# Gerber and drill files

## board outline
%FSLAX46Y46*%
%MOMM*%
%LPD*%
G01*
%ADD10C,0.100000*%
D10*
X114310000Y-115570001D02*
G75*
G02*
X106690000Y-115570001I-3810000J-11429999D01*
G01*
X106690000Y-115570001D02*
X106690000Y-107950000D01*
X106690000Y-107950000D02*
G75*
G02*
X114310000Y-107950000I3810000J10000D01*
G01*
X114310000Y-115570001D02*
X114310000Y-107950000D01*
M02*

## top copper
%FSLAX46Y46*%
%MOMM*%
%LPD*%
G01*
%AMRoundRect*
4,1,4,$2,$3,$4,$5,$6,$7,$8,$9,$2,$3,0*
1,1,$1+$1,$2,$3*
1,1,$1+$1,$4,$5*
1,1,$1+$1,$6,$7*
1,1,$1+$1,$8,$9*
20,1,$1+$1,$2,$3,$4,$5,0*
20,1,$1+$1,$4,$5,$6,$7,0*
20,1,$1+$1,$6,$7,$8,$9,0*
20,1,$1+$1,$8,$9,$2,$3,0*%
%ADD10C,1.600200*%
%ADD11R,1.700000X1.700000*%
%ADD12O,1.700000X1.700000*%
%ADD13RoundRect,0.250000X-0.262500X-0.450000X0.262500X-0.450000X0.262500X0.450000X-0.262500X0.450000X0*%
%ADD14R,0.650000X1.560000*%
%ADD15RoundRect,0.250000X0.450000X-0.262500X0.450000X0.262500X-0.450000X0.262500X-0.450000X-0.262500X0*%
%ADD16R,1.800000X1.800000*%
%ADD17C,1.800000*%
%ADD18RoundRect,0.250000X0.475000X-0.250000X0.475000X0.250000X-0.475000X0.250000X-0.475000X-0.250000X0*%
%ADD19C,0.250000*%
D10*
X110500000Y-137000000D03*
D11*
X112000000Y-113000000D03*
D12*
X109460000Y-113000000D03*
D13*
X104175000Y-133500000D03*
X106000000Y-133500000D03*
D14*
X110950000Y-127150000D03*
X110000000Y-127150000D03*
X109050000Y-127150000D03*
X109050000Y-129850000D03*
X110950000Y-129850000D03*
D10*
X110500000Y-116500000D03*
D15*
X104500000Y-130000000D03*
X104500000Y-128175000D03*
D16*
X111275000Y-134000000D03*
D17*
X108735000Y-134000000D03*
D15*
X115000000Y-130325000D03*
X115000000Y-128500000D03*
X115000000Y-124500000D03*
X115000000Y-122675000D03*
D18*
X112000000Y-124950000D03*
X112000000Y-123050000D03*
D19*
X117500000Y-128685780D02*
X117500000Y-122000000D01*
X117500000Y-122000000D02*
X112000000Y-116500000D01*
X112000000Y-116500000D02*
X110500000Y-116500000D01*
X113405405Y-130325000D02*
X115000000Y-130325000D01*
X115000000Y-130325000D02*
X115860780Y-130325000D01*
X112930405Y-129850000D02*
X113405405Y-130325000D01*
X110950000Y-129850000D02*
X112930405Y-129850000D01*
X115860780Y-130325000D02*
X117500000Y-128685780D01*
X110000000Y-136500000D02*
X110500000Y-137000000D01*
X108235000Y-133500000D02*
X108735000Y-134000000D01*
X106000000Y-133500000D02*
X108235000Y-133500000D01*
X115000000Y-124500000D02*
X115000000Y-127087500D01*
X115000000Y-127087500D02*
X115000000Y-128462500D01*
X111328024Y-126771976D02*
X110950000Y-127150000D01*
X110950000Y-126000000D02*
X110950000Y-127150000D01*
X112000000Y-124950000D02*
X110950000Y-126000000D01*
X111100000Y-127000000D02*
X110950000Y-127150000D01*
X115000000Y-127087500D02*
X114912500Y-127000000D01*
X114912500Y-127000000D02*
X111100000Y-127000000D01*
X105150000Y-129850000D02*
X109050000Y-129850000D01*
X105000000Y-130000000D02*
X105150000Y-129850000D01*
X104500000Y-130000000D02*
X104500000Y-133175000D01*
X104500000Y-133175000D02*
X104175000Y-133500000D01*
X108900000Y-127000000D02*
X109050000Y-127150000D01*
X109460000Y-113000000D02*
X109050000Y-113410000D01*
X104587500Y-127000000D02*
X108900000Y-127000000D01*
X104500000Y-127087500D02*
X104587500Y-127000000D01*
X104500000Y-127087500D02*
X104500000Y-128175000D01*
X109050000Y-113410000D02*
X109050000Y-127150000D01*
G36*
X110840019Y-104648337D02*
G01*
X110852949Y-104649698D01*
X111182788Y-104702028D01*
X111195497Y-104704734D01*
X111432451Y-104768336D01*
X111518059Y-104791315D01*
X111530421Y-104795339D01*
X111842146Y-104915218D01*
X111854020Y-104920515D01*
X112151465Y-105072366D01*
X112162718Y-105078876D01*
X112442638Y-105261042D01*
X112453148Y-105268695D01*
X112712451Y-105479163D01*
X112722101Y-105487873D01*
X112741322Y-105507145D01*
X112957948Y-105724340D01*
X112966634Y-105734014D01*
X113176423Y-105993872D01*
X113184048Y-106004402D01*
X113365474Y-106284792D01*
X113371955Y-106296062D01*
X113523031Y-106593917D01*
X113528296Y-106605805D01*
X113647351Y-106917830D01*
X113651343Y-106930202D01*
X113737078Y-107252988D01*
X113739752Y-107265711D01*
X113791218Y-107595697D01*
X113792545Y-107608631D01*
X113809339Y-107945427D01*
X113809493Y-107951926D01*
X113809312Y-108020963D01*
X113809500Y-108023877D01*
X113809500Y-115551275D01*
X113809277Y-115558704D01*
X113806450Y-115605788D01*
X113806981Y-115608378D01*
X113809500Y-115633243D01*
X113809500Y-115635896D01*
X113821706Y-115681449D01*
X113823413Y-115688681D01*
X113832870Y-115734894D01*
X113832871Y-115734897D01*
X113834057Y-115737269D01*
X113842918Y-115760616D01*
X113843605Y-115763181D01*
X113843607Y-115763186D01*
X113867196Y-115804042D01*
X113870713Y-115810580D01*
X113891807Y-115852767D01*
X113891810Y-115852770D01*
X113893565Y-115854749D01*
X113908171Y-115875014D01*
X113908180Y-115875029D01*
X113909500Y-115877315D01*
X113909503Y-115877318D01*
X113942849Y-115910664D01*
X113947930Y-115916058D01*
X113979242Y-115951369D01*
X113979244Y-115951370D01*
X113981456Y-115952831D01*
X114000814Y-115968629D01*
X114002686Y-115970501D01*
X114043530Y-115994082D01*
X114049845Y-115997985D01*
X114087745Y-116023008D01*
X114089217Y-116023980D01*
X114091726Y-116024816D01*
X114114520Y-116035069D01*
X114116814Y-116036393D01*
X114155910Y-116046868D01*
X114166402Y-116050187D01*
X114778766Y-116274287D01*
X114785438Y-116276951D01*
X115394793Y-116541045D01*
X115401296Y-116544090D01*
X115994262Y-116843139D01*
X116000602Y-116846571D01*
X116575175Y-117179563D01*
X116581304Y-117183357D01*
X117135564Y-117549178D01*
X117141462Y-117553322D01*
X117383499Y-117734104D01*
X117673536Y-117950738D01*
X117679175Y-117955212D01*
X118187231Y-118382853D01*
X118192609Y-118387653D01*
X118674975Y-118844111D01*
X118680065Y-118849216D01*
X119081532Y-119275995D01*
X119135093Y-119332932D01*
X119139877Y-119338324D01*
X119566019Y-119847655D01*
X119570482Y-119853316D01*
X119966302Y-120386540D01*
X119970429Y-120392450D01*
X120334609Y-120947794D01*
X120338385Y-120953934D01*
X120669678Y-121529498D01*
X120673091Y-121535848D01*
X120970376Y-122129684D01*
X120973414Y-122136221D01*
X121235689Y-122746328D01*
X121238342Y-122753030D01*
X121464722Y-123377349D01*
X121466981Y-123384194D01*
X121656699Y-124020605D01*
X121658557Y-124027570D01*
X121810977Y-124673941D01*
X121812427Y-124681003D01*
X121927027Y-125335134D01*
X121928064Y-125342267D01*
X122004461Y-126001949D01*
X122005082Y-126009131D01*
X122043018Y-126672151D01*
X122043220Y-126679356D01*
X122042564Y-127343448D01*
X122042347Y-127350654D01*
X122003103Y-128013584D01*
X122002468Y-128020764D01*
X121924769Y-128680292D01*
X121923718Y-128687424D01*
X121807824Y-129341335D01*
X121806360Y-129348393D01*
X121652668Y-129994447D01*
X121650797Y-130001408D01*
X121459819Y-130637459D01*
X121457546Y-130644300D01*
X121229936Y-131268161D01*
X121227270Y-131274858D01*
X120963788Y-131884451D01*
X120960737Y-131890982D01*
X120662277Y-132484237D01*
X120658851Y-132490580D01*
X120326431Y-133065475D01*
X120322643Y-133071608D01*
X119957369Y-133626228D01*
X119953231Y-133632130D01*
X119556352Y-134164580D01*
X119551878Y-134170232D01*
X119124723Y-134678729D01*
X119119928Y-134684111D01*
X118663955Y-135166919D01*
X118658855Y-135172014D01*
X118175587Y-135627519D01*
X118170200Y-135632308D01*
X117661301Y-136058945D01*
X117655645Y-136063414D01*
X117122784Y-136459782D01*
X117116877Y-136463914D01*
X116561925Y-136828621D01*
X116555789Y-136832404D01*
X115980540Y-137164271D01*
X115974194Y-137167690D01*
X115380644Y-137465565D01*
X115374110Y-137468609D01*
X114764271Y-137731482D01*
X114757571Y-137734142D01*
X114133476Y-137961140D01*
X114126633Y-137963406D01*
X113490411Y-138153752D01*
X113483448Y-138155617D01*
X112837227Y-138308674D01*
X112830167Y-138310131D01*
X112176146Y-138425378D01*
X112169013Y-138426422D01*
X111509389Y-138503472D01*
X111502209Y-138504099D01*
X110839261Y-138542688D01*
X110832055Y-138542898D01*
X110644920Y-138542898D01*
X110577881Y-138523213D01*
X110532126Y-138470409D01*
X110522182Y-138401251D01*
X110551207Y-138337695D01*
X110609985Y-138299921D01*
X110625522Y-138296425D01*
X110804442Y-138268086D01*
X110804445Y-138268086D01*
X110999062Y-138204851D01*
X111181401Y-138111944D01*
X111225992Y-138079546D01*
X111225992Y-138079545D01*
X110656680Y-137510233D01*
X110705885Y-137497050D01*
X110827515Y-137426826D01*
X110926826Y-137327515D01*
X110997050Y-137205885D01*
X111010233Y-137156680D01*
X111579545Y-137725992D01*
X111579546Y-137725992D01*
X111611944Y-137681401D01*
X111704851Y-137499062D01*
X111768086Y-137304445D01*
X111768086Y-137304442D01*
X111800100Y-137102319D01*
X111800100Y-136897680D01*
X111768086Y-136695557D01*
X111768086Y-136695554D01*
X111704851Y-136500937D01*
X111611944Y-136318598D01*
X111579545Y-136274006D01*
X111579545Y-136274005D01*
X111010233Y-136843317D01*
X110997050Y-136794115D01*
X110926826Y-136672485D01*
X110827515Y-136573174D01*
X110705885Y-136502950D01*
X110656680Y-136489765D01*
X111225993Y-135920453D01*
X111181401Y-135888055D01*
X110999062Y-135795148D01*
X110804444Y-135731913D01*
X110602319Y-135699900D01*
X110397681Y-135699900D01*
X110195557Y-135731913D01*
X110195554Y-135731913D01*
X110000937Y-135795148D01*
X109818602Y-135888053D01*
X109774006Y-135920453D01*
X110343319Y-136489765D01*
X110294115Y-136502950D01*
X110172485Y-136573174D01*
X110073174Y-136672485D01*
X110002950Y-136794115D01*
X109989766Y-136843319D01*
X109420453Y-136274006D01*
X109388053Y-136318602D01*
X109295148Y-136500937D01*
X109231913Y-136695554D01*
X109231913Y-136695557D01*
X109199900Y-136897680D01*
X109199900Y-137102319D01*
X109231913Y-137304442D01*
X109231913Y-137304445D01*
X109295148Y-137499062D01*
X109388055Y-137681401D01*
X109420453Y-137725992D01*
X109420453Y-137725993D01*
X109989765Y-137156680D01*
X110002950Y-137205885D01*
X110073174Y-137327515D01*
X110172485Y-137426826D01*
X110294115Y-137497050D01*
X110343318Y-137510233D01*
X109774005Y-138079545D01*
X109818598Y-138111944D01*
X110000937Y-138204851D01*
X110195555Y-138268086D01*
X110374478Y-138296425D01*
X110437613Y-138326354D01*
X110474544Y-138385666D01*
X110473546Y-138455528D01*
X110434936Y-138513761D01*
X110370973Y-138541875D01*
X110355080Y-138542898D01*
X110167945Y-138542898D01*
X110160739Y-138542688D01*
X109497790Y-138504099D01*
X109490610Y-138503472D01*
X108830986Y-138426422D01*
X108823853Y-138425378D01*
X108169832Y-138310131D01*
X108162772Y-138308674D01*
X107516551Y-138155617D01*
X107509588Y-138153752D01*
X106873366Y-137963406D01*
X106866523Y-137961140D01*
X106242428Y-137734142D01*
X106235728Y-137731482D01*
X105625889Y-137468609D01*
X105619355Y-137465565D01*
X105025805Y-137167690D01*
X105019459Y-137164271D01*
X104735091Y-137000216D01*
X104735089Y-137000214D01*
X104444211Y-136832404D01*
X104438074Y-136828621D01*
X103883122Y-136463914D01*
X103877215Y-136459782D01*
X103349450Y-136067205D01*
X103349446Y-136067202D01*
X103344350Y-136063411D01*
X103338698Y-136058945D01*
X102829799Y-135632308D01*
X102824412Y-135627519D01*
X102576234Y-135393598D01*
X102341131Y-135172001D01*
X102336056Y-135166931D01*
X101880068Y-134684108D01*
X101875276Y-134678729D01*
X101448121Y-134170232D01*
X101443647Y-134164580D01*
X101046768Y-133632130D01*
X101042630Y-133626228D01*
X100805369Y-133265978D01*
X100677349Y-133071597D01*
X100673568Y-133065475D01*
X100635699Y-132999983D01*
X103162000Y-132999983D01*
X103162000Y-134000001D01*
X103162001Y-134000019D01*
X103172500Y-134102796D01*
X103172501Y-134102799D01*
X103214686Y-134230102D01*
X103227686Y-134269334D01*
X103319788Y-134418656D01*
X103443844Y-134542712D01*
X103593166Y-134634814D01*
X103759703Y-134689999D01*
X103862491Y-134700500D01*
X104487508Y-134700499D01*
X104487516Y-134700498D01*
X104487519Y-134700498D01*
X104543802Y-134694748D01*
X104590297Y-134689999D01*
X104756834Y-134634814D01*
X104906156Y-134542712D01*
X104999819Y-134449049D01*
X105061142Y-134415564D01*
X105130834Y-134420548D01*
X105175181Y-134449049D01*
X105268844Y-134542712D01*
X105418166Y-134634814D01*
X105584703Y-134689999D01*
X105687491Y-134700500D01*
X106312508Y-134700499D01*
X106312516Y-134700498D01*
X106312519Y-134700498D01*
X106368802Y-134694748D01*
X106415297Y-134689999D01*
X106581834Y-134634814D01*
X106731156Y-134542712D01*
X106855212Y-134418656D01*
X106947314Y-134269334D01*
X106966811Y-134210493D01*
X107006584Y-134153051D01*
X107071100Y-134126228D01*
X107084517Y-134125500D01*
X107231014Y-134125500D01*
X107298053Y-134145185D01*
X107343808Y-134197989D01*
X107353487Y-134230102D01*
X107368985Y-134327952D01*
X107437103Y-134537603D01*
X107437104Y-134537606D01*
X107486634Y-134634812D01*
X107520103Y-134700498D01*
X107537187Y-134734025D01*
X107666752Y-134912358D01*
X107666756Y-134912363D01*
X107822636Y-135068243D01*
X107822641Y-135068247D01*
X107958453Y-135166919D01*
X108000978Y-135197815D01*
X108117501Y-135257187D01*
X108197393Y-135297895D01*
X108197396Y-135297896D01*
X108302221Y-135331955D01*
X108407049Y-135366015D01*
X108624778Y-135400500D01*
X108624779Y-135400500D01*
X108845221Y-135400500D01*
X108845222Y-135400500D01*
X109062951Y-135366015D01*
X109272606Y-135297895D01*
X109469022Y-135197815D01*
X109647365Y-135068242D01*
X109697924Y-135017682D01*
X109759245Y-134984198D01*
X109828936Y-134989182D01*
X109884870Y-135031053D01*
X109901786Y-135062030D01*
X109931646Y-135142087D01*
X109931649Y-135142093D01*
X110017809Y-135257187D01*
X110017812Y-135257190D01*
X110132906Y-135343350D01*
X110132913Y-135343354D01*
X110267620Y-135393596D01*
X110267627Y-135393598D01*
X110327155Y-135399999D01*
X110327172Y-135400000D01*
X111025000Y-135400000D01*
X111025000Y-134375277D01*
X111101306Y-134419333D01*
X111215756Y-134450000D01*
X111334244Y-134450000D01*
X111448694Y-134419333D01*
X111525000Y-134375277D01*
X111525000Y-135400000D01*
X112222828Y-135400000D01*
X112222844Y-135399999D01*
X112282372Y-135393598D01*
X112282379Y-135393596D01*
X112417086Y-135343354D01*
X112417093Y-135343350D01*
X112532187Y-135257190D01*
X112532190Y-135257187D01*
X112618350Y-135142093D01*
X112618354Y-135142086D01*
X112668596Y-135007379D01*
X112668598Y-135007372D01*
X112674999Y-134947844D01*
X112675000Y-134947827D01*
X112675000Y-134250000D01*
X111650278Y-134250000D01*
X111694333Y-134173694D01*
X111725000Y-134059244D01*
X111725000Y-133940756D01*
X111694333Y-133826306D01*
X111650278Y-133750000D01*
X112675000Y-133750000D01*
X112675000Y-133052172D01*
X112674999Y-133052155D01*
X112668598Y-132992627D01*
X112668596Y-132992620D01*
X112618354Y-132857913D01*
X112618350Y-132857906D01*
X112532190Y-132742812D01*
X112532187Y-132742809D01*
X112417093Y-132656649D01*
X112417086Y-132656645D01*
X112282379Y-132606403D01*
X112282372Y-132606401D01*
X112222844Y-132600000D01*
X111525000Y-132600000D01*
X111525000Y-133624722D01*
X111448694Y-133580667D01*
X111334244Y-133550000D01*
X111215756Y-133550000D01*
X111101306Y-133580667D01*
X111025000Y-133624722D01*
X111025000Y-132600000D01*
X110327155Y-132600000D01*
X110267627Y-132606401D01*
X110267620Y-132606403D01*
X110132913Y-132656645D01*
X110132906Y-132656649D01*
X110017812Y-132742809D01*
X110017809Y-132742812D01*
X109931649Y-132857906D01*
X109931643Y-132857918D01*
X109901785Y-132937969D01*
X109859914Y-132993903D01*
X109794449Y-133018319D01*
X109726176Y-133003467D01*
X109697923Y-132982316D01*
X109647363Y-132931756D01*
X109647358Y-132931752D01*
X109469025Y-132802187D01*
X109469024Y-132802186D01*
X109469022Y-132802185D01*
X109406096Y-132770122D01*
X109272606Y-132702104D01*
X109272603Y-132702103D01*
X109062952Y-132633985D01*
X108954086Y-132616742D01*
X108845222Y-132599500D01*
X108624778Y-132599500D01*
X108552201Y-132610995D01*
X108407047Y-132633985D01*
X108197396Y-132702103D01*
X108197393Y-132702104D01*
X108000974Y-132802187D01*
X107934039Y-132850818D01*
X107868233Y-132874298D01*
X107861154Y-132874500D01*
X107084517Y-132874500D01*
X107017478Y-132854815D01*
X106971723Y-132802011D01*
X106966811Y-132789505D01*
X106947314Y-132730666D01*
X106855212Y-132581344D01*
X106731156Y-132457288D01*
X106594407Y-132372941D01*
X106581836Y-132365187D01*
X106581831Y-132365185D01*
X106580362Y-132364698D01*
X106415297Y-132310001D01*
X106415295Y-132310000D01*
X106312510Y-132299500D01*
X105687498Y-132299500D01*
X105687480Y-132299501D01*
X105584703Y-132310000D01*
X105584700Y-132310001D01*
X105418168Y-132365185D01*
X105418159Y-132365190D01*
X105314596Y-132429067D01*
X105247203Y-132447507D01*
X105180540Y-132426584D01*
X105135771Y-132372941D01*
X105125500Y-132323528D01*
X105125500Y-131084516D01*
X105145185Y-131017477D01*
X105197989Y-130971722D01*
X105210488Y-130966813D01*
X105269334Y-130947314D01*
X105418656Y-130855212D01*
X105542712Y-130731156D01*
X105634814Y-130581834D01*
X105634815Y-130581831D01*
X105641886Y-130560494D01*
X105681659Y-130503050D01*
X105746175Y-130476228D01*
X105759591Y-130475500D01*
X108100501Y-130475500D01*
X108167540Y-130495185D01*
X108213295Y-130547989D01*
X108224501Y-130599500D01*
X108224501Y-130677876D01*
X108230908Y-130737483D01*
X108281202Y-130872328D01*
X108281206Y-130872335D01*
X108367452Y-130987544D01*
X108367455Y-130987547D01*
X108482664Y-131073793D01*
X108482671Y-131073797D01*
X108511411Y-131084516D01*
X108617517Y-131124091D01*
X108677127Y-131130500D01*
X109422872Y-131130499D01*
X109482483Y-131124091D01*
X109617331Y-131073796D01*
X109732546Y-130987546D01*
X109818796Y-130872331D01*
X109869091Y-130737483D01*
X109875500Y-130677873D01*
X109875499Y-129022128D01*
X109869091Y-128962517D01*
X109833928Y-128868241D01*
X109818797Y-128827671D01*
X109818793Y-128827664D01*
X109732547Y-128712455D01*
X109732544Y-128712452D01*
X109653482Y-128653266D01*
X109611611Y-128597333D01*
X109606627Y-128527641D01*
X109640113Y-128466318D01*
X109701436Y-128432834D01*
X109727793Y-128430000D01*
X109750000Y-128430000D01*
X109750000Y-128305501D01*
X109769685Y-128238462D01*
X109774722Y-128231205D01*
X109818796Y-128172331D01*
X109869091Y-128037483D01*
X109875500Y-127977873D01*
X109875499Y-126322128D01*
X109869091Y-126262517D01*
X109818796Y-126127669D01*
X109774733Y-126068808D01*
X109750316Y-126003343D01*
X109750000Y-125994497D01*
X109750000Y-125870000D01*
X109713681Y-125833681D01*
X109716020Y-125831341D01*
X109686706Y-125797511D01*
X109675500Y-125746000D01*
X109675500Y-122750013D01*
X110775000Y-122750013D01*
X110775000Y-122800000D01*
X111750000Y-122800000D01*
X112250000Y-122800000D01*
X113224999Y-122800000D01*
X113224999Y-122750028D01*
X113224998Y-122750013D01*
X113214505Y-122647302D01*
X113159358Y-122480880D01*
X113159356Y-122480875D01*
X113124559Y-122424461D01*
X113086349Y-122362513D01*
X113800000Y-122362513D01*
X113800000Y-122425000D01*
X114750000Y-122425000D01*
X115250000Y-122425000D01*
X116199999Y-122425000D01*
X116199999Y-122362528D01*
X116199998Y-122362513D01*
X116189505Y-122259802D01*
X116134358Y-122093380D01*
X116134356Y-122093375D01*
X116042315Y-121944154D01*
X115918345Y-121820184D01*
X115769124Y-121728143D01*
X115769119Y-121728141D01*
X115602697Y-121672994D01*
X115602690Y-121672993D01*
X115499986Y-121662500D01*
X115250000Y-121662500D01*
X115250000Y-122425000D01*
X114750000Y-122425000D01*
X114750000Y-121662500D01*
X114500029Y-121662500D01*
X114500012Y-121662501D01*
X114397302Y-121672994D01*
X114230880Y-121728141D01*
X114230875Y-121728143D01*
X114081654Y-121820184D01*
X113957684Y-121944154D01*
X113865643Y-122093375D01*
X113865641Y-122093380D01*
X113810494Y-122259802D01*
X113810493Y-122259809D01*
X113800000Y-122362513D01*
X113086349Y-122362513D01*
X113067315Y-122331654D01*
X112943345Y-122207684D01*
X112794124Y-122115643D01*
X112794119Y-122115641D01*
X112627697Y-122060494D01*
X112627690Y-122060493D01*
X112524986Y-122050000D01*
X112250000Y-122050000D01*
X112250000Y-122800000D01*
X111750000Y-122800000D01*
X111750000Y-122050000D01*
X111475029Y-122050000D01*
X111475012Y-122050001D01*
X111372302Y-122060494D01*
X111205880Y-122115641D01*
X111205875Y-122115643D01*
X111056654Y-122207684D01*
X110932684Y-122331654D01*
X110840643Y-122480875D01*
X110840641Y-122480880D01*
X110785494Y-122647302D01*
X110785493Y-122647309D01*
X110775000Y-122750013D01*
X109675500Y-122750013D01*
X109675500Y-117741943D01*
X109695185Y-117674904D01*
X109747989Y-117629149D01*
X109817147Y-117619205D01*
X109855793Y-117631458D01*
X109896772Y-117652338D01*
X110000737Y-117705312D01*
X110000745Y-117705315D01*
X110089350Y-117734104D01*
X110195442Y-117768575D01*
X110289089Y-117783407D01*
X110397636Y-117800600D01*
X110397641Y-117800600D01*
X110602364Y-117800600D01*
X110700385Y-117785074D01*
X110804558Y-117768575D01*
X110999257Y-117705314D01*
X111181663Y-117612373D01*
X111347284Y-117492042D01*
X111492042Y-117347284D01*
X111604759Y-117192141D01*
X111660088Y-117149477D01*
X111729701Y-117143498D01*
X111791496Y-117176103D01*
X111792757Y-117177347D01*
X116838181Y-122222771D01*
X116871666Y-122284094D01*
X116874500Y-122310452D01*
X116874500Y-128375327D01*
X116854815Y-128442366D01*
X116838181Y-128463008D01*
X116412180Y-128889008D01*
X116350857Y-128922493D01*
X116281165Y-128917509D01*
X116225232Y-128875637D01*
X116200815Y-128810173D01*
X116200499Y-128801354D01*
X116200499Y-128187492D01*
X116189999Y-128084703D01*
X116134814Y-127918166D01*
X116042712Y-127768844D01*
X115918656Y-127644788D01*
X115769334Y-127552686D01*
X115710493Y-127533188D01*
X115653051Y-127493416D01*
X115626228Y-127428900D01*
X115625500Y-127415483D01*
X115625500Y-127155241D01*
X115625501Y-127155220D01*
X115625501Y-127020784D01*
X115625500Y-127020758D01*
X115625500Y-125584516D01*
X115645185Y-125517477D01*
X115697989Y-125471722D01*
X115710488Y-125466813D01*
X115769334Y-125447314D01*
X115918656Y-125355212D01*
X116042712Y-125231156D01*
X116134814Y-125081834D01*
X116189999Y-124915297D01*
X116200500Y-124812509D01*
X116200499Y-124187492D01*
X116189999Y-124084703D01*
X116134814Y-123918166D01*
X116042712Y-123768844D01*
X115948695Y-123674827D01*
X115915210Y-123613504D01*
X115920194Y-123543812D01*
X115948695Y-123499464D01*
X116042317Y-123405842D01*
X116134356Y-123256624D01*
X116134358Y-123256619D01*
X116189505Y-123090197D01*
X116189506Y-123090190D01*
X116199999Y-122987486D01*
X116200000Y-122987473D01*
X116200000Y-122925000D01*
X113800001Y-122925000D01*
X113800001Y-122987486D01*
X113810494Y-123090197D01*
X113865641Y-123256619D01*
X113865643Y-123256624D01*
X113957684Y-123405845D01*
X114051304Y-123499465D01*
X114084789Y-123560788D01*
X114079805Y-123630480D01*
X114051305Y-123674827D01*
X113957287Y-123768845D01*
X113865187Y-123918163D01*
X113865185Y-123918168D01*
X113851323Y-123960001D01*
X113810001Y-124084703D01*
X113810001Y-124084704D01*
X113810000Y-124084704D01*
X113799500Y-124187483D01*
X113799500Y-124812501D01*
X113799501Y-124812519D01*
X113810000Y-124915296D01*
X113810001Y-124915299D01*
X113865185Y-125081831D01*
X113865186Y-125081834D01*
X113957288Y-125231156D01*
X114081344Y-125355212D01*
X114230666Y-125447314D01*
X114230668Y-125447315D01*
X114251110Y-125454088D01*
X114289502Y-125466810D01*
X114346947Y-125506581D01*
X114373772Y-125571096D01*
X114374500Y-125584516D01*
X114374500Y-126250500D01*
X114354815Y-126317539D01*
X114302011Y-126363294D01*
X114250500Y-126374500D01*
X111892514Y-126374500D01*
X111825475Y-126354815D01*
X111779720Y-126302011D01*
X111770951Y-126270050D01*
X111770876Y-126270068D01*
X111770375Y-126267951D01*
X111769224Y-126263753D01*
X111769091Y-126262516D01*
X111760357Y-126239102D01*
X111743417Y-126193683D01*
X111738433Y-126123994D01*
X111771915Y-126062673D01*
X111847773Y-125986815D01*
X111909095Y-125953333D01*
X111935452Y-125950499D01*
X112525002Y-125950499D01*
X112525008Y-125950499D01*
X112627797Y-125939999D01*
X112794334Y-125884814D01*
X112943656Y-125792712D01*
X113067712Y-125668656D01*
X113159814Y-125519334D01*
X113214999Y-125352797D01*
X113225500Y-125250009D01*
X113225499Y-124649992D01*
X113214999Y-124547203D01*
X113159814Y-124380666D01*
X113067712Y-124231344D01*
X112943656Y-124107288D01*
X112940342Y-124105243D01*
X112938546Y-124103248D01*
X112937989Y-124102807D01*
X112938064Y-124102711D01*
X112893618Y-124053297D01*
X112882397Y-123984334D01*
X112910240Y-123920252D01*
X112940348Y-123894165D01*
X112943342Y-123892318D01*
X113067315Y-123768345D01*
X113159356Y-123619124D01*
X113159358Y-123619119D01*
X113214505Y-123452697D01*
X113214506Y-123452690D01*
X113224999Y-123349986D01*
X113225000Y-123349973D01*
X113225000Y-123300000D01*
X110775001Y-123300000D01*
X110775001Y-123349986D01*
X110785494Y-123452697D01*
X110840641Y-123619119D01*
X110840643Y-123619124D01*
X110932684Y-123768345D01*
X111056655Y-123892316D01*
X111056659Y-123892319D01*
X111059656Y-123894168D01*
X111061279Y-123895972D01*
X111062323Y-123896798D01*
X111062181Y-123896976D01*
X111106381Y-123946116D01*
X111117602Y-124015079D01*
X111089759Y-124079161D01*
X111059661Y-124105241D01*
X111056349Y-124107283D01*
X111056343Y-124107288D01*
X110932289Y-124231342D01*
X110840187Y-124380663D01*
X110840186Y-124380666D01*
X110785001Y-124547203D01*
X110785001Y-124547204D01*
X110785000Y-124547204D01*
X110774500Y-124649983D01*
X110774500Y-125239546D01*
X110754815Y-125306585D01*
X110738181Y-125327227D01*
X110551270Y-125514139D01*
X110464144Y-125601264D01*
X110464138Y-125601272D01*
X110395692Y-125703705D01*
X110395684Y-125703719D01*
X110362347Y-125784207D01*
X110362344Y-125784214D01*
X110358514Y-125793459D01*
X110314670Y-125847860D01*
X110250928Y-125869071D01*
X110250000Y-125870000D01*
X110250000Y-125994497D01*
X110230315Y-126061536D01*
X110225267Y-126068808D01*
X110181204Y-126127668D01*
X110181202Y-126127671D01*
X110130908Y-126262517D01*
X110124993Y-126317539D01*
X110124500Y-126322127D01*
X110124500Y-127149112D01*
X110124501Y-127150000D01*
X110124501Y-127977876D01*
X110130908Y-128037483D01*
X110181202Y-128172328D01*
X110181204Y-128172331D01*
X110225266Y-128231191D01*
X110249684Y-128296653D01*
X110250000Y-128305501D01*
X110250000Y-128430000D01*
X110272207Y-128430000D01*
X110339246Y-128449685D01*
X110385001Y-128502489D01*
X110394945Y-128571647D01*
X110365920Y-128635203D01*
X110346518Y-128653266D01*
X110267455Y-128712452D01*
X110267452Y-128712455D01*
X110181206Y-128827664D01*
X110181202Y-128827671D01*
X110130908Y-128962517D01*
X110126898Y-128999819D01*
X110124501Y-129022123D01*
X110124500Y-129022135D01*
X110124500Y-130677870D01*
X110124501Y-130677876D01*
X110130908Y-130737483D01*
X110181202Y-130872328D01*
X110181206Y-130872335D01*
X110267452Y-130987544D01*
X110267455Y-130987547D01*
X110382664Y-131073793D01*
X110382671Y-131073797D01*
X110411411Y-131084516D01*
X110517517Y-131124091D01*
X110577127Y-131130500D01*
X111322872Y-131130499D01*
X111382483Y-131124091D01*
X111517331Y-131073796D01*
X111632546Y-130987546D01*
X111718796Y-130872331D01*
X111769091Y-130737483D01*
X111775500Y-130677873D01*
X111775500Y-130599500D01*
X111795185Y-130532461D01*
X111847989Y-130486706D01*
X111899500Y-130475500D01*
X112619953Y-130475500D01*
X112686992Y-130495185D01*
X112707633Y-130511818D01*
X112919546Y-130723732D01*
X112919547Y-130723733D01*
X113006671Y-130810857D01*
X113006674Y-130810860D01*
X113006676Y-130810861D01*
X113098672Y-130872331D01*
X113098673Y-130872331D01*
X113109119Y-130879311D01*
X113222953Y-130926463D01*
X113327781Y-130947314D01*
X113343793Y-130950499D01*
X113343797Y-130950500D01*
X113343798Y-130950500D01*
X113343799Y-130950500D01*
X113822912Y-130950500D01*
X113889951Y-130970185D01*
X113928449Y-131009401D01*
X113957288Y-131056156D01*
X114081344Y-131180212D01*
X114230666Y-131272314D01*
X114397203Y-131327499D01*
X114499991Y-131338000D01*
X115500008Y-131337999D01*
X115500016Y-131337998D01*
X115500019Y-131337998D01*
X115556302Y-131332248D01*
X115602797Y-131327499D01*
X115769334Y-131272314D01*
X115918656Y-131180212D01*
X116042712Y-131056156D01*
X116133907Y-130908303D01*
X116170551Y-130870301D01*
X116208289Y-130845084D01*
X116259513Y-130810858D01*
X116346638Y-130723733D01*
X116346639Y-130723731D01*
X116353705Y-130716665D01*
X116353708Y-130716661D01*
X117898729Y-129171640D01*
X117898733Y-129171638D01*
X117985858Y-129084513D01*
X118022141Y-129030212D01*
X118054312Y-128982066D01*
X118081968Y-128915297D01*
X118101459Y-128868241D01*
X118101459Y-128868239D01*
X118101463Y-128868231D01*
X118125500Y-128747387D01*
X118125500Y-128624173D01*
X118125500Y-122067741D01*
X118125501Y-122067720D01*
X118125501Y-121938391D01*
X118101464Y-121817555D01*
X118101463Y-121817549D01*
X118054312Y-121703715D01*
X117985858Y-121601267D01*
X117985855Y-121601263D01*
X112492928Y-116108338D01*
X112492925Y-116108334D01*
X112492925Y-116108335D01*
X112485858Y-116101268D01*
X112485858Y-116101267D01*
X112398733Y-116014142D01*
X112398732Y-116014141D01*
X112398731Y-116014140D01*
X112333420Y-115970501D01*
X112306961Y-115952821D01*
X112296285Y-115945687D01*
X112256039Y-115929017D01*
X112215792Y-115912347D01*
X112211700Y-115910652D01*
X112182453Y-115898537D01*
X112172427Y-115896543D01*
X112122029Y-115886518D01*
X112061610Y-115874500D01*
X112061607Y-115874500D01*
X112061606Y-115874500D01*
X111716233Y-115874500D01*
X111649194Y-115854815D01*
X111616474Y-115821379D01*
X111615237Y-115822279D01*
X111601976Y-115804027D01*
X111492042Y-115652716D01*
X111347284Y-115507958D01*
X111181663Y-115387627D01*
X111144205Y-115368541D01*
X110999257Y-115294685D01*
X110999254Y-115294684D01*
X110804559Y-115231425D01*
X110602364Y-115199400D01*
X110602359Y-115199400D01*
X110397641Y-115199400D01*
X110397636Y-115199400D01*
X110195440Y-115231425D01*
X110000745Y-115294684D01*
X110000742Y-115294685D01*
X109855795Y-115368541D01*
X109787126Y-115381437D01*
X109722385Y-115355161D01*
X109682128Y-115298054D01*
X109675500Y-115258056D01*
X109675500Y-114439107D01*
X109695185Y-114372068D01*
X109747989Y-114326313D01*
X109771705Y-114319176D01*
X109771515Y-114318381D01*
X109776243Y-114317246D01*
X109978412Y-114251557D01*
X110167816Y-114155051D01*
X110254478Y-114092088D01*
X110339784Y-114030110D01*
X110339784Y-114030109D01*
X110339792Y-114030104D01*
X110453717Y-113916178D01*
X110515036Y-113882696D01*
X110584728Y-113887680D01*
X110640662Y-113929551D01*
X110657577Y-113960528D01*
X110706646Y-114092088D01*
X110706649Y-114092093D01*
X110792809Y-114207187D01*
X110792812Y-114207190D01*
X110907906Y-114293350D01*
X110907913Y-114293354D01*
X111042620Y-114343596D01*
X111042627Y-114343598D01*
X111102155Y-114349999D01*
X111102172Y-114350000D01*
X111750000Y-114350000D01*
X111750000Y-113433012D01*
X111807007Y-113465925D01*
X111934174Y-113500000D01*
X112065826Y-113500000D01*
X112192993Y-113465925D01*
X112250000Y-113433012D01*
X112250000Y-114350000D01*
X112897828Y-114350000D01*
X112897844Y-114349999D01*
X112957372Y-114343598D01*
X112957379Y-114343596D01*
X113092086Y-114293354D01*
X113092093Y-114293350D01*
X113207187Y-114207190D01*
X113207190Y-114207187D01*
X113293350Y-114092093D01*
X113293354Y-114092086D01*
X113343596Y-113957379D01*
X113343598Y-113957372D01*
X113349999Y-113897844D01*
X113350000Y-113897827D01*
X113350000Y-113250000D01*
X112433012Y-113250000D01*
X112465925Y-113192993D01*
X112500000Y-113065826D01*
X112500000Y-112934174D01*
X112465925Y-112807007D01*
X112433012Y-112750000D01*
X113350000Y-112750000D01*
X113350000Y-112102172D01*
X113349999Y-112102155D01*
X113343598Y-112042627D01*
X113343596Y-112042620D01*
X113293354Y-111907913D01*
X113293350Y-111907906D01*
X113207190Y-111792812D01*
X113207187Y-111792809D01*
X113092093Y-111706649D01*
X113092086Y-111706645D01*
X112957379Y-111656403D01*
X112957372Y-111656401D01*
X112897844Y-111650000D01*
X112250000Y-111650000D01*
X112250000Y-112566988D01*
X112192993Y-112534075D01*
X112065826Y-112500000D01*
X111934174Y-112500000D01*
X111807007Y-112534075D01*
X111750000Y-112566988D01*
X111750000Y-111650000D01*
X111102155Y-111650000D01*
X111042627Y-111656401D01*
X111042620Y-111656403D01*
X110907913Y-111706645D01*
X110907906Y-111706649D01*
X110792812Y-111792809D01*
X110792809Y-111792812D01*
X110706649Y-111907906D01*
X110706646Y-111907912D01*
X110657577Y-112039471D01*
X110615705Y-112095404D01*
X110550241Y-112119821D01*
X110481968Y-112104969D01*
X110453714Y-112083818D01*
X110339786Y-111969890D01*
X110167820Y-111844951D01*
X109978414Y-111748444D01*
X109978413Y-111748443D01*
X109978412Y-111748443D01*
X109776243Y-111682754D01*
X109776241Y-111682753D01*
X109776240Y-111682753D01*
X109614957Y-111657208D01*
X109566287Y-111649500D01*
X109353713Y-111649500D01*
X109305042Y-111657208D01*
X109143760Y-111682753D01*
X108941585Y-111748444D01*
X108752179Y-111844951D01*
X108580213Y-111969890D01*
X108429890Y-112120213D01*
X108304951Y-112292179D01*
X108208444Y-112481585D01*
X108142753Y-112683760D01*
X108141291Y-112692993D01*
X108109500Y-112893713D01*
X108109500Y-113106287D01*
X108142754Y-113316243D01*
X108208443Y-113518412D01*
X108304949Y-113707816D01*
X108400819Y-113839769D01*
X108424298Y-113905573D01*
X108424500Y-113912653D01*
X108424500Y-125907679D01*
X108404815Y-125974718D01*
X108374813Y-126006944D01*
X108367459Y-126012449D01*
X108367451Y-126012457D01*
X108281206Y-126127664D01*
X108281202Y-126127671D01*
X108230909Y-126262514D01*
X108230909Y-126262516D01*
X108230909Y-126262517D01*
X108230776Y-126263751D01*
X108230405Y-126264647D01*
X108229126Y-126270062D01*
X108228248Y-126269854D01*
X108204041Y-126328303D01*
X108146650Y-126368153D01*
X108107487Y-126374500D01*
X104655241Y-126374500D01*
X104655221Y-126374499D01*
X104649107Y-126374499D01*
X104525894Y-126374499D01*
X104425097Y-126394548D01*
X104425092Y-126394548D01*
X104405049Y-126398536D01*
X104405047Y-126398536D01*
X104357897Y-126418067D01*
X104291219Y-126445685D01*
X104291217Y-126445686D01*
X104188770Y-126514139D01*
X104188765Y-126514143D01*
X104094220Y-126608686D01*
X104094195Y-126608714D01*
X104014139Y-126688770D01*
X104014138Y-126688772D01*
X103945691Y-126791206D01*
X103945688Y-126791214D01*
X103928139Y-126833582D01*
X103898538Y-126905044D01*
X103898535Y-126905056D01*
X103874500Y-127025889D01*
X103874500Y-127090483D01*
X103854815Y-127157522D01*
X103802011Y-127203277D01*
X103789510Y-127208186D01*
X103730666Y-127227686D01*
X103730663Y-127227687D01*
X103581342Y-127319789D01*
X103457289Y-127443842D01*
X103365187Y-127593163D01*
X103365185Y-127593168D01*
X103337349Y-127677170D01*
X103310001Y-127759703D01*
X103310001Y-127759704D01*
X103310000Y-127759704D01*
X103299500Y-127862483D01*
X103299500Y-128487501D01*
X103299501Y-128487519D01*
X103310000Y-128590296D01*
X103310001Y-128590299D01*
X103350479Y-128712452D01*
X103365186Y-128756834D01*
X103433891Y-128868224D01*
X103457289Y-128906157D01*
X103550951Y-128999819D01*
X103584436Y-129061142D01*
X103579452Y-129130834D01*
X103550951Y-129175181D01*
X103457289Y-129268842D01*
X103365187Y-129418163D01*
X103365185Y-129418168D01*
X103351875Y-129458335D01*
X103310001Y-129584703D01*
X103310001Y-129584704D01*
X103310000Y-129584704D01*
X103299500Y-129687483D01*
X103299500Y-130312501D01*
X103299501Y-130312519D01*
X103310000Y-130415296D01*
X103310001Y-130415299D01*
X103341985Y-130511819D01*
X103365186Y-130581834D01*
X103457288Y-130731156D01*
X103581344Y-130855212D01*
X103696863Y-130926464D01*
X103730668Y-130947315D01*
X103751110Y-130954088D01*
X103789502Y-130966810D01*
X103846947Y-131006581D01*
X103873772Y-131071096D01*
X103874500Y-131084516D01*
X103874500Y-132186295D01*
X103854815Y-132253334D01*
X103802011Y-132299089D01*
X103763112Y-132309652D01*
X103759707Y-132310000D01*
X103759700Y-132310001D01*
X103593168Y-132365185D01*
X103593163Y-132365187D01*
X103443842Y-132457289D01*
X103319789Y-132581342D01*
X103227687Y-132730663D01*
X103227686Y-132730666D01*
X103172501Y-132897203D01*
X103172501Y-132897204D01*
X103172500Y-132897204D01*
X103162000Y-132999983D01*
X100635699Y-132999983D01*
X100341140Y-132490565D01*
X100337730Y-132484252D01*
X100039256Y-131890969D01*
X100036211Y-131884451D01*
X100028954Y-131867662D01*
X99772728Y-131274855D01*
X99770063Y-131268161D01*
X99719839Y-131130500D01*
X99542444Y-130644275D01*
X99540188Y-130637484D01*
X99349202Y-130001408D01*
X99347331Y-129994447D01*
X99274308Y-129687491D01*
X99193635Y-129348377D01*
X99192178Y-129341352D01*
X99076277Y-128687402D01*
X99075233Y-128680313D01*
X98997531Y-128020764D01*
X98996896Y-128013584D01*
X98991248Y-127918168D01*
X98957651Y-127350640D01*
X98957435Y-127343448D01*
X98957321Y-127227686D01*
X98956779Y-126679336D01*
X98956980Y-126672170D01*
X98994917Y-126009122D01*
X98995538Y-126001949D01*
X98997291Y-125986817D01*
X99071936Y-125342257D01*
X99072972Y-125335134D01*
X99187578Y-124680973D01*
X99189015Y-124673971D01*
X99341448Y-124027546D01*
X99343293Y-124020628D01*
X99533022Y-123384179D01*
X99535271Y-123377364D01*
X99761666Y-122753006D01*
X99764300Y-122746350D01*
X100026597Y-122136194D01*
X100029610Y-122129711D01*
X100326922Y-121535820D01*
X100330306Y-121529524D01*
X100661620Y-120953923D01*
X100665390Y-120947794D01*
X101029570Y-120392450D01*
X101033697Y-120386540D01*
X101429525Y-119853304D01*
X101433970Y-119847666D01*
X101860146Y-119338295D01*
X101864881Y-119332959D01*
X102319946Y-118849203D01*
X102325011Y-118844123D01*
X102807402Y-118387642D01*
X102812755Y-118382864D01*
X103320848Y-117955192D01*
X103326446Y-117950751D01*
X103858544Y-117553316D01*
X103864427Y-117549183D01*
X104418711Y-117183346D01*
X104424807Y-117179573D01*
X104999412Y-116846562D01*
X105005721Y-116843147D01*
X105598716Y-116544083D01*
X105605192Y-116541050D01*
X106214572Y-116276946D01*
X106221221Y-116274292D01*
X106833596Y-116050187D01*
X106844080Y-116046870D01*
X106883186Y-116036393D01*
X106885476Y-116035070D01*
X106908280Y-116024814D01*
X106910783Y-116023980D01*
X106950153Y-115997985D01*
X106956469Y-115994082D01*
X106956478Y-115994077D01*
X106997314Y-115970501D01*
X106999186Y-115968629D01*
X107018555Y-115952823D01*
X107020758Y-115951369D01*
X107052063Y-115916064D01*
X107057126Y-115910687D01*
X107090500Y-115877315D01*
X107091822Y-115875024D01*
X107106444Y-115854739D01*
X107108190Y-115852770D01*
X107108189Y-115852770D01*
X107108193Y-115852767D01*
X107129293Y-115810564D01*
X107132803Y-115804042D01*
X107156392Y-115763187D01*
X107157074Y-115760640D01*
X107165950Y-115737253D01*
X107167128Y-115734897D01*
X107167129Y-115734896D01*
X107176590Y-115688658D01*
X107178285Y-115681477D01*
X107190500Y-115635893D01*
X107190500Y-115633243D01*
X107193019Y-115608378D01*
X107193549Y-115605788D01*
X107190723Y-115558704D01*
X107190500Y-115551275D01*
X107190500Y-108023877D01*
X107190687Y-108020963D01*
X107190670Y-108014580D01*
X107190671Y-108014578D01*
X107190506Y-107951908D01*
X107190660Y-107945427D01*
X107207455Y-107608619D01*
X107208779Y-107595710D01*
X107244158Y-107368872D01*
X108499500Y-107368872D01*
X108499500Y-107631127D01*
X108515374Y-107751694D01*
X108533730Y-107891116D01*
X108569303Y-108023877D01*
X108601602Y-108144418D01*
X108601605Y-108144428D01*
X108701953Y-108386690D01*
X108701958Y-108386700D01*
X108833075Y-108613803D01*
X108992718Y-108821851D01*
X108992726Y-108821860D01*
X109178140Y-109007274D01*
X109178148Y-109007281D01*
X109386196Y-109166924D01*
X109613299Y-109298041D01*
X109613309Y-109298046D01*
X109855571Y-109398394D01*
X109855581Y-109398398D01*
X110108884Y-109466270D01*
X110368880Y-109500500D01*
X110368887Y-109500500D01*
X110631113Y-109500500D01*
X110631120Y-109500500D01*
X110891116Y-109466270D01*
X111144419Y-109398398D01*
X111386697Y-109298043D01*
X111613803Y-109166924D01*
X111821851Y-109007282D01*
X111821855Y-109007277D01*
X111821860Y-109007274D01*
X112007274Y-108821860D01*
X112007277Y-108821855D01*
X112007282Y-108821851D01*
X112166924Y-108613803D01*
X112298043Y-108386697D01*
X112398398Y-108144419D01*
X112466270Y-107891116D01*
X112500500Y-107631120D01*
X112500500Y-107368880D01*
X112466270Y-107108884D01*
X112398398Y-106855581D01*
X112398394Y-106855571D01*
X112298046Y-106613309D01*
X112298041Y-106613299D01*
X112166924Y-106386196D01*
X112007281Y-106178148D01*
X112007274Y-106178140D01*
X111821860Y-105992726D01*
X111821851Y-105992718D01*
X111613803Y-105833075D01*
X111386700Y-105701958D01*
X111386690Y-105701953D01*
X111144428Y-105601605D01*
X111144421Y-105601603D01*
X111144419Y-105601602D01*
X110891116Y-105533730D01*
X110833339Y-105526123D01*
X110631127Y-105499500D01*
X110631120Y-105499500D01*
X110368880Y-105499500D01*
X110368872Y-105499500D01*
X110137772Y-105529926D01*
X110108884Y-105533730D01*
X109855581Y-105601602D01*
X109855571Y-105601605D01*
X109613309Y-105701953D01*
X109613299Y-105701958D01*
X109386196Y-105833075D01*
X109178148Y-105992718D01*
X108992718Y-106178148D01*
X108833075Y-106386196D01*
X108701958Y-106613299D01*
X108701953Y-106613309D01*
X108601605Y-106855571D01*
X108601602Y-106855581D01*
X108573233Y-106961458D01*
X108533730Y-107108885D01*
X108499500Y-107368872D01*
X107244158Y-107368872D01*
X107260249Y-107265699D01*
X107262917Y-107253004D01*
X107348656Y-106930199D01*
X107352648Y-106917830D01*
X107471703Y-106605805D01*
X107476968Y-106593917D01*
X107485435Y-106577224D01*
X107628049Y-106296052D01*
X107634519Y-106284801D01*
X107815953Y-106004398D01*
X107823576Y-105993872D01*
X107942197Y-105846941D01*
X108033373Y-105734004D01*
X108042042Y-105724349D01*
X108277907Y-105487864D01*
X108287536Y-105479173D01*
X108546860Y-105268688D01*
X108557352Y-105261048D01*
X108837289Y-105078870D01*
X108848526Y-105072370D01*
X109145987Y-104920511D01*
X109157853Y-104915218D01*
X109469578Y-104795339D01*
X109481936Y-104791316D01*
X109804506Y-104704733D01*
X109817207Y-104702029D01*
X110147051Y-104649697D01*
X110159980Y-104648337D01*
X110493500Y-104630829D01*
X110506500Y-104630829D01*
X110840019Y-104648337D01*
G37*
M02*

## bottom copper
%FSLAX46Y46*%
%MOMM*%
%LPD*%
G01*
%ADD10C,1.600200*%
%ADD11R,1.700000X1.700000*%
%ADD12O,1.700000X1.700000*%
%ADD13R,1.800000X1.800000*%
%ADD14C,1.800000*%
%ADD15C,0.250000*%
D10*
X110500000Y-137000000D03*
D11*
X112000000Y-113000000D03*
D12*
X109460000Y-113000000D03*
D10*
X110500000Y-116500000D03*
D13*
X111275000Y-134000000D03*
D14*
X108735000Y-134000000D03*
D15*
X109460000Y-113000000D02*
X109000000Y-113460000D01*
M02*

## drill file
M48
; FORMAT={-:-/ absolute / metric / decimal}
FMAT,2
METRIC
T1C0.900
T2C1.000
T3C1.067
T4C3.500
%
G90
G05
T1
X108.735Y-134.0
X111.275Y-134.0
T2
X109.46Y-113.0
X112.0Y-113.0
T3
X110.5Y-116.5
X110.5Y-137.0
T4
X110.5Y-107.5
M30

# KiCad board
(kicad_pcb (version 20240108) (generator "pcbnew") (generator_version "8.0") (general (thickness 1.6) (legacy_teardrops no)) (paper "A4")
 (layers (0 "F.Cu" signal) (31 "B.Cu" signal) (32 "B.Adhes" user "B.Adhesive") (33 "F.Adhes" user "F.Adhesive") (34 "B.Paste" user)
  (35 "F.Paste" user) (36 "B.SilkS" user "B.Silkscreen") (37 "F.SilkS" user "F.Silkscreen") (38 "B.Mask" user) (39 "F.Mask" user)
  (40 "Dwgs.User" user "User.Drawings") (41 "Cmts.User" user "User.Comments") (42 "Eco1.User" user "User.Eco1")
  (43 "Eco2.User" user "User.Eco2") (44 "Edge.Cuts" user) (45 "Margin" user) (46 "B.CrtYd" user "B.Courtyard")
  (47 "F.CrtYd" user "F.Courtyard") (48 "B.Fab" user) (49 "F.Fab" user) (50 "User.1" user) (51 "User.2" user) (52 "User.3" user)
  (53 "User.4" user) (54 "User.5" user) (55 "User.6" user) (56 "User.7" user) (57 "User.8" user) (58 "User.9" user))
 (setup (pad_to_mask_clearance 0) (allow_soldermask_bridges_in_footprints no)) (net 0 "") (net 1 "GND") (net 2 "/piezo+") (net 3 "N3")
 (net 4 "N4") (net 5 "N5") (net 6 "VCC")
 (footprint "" (layer "F.Cu") (at 110.5 137)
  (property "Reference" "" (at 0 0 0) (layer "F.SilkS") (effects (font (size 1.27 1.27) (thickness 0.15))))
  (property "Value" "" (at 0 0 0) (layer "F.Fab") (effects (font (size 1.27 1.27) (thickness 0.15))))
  (pad "2" thru_hole circle (at 0 0) (size 1.6002 1.6002) (drill 1.0668) (layers "*.Cu" "*.Mask") (remove_unused_layers no) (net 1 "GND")
   (solder_mask_margin 0.102)))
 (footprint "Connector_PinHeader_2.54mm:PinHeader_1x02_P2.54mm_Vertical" (layer "F.Cu") (at 112 113 -90)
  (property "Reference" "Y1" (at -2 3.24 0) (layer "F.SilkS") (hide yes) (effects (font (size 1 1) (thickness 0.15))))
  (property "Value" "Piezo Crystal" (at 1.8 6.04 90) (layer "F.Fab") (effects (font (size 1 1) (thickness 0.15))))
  (pad "1" thru_hole rect (at 0 0 270) (size 1.7 1.7) (drill 1) (layers "*.Cu" "*.Mask") (remove_unused_layers no) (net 1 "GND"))
  (pad "2" thru_hole oval (at 0 2.54 270) (size 1.7 1.7) (drill 1) (layers "*.Cu" "*.Mask") (remove_unused_layers no) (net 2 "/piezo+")))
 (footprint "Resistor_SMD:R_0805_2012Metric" (layer "F.Cu") (at 105.0875 133.5)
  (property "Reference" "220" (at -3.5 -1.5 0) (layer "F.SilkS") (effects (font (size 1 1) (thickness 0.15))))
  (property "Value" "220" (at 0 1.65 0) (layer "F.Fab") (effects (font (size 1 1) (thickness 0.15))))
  (pad "1" smd roundrect (at -0.9125 0) (size 1.025 1.4) (layers "F.Cu" "F.Paste" "F.Mask") (roundrect_rratio 0.243902439) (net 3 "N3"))
  (pad "2" smd roundrect (at 0.9125 0) (size 1.025 1.4) (layers "F.Cu" "F.Paste" "F.Mask") (roundrect_rratio 0.243902439) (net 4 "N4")))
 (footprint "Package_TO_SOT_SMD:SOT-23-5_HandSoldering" (layer "F.Cu") (at 110 128.5 -90)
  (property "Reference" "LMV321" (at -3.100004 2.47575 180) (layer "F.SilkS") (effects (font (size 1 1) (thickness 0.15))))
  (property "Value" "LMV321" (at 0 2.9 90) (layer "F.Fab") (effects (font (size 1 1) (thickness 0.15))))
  (pad "1" smd rect (at -1.35 -0.95 270) (size 1.56 0.65) (layers "F.Cu" "F.Paste" "F.Mask") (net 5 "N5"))
  (pad "2" smd rect (at -1.35 0 270) (size 1.56 0.65) (layers "F.Cu" "F.Paste" "F.Mask") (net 1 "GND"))
  (pad "3" smd rect (at -1.35 0.95 270) (size 1.56 0.65) (layers "F.Cu" "F.Paste" "F.Mask") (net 2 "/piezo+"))
  (pad "4" smd rect (at 1.35 0.95 270) (size 1.56 0.65) (layers "F.Cu" "F.Paste" "F.Mask") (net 3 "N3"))
  (pad "5" smd rect (at 1.35 -0.95 270) (size 1.56 0.65) (layers "F.Cu" "F.Paste" "F.Mask") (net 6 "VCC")))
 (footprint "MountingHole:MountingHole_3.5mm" (layer "F.Cu") (at 110.5 107.5)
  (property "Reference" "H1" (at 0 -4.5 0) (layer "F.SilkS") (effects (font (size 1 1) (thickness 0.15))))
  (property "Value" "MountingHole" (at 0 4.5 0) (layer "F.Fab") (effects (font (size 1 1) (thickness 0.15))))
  (pad "" np_thru_hole circle (at 0 0) (size 3.5 3.5) (drill 3.5) (layers "*.Cu" "*.Mask")))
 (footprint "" (layer "F.Cu") (at 110.5 116.5)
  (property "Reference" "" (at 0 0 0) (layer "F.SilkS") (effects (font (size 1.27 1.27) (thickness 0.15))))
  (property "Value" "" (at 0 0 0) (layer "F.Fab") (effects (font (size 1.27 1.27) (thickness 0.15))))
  (pad "1" thru_hole circle (at 0 0) (size 1.6002 1.6002) (drill 1.0668) (layers "*.Cu" "*.Mask") (remove_unused_layers no) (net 6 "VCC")
   (solder_mask_margin 0.102)))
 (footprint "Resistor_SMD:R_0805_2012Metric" (layer "F.Cu") (at 104.5 129.0875 90)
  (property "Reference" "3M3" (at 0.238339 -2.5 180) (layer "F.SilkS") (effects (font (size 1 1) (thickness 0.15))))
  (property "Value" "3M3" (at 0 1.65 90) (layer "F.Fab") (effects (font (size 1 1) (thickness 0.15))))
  (pad "1" smd roundrect (at -0.9125 0 90) (size 1.025 1.4) (layers "F.Cu" "F.Paste" "F.Mask") (roundrect_rratio 0.243902439) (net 3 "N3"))
  (pad "2" smd roundrect (at 0.9125 0 90) (size 1.025 1.4) (layers "F.Cu" "F.Paste" "F.Mask") (roundrect_rratio 0.243902439)
   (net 2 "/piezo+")))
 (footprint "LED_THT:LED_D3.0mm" (layer "F.Cu") (at 111.275 134 180)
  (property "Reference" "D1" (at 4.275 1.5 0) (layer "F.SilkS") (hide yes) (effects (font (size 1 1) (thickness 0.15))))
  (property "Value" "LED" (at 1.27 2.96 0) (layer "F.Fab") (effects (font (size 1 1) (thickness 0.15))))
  (pad "1" thru_hole rect (at 0 0 180) (size 1.8 1.8) (drill 0.9) (layers "*.Cu" "*.Mask") (remove_unused_layers no) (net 1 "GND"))
  (pad "2" thru_hole circle (at 2.54 0 180) (size 1.8 1.8) (drill 0.9) (layers "*.Cu" "*.Mask") (remove_unused_layers no) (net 4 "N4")))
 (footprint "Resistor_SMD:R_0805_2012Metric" (layer "F.Cu") (at 115 129.4125 90)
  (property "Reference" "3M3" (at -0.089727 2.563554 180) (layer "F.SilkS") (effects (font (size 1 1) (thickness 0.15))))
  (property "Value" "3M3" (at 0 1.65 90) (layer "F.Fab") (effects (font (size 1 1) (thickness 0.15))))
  (pad "1" smd roundrect (at -0.9125 0 90) (size 1.025 1.4) (layers "F.Cu" "F.Paste" "F.Mask") (roundrect_rratio 0.243902439) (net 6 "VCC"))
  (pad "2" smd roundrect (at 0.9125 0 90) (size 1.025 1.4) (layers "F.Cu" "F.Paste" "F.Mask") (roundrect_rratio 0.243902439) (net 5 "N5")))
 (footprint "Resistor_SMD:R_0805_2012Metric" (layer "F.Cu") (at 115 123.5875 90)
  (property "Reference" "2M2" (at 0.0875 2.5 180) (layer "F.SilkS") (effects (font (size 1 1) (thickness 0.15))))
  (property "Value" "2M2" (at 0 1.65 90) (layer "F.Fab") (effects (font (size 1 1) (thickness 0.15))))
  (pad "1" smd roundrect (at -0.9125 0 90) (size 1.025 1.4) (layers "F.Cu" "F.Paste" "F.Mask") (roundrect_rratio 0.243902439) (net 5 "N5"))
  (pad "2" smd roundrect (at 0.9125 0 90) (size 1.025 1.4) (layers "F.Cu" "F.Paste" "F.Mask") (roundrect_rratio 0.243902439) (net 1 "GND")))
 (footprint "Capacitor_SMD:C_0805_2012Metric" (layer "F.Cu") (at 112 124 90)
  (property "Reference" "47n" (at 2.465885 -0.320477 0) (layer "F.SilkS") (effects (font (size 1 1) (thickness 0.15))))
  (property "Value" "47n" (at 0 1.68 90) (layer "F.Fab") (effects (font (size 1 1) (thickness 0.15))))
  (pad "1" smd roundrect (at -0.95 0 90) (size 1 1.45) (layers "F.Cu" "F.Paste" "F.Mask") (roundrect_rratio 0.25) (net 5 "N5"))
  (pad "2" smd roundrect (at 0.95 0 90) (size 1 1.45) (layers "F.Cu" "F.Paste" "F.Mask") (roundrect_rratio 0.25) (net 1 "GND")))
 (gr_arc (start 114.31 115.570001) (mid 110.5 139.048277) (end 106.69 115.570001) (stroke (width 0.1) (type default)) (layer "Edge.Cuts"))
 (gr_line (start 106.69 115.570001) (end 106.69 107.95) (stroke (width 0.1) (type default)) (layer "Edge.Cuts"))
 (gr_arc (start 106.69 107.95) (mid 110.5 104.129987) (end 114.31 107.95) (stroke (width 0.1) (type default)) (layer "Edge.Cuts"))
 (gr_line (start 114.31 115.570001) (end 114.31 107.95) (stroke (width 0.1) (type default)) (layer "Edge.Cuts"))
 (segment (start 117.5 128.68578) (end 117.5 122) (width 0.25) (layer "F.Cu") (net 6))
 (segment (start 117.5 122) (end 112 116.5) (width 0.25) (layer "F.Cu") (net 6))
 (segment (start 112 116.5) (end 110.5 116.5) (width 0.25) (layer "F.Cu") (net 6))
 (segment (start 113.405405 130.325) (end 115 130.325) (width 0.25) (layer "F.Cu") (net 6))
 (segment (start 115 130.325) (end 115.86078 130.325) (width 0.25) (layer "F.Cu") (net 6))
 (segment (start 112.930405 129.85) (end 113.405405 130.325) (width 0.25) (layer "F.Cu") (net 6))
 (segment (start 110.95 129.85) (end 112.930405 129.85) (width 0.25) (layer "F.Cu") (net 6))
 (segment (start 115.86078 130.325) (end 117.5 128.68578) (width 0.25) (layer "F.Cu") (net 6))
 (segment (start 110 136.5) (end 110.5 137) (width 0.25) (layer "F.Cu") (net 1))
 (segment (start 108.235 133.5) (end 108.735 134) (width 0.25) (layer "F.Cu") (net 4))
 (segment (start 106 133.5) (end 108.235 133.5) (width 0.25) (layer "F.Cu") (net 4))
 (segment (start 115 124.5) (end 115 127.0875) (width 0.25) (layer "F.Cu") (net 5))
 (segment (start 115 127.0875) (end 115 128.4625) (width 0.25) (layer "F.Cu") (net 5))
 (segment (start 111.328024 126.771976) (end 110.95 127.15) (width 0.25) (layer "F.Cu") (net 5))
 (segment (start 110.95 126) (end 110.95 127.15) (width 0.25) (layer "F.Cu") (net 5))
 (segment (start 112 124.95) (end 110.95 126) (width 0.25) (layer "F.Cu") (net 5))
 (segment (start 111.1 127) (end 110.95 127.15) (width 0.25) (layer "F.Cu") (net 5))
 (segment (start 115 127.0875) (end 114.9125 127) (width 0.25) (layer "F.Cu") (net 5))
 (segment (start 114.9125 127) (end 111.1 127) (width 0.25) (layer "F.Cu") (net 5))
 (segment (start 105.15 129.85) (end 109.05 129.85) (width 0.25) (layer "F.Cu") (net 3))
 (segment (start 105 130) (end 105.15 129.85) (width 0.25) (layer "F.Cu") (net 3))
 (segment (start 104.5 130) (end 104.5 133.175) (width 0.25) (layer "F.Cu") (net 3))
 (segment (start 104.5 133.175) (end 104.175 133.5) (width 0.25) (layer "F.Cu") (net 3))
 (segment (start 108.9 127) (end 109.05 127.15) (width 0.25) (layer "F.Cu") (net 2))
 (segment (start 109.46 113) (end 109.05 113.41) (width 0.25) (layer "F.Cu") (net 2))
 (segment (start 104.5875 127) (end 108.9 127) (width 0.25) (layer "F.Cu") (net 2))
 (segment (start 104.5 127.0875) (end 104.5875 127) (width 0.25) (layer "F.Cu") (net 2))
 (segment (start 104.5 127.0875) (end 104.5 128.175) (width 0.25) (layer "F.Cu") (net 2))
 (segment (start 109.05 113.41) (end 109.05 127.15) (width 0.25) (layer "F.Cu") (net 2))
 (segment (start 109.46 113) (end 109 113.46) (width 0.25) (layer "B.Cu") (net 2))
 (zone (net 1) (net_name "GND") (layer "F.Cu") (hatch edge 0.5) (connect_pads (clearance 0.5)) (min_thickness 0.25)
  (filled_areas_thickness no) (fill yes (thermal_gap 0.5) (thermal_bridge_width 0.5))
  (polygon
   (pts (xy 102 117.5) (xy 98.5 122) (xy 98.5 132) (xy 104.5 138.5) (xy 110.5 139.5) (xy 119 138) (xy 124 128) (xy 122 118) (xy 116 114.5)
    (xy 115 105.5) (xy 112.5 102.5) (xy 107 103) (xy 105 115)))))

